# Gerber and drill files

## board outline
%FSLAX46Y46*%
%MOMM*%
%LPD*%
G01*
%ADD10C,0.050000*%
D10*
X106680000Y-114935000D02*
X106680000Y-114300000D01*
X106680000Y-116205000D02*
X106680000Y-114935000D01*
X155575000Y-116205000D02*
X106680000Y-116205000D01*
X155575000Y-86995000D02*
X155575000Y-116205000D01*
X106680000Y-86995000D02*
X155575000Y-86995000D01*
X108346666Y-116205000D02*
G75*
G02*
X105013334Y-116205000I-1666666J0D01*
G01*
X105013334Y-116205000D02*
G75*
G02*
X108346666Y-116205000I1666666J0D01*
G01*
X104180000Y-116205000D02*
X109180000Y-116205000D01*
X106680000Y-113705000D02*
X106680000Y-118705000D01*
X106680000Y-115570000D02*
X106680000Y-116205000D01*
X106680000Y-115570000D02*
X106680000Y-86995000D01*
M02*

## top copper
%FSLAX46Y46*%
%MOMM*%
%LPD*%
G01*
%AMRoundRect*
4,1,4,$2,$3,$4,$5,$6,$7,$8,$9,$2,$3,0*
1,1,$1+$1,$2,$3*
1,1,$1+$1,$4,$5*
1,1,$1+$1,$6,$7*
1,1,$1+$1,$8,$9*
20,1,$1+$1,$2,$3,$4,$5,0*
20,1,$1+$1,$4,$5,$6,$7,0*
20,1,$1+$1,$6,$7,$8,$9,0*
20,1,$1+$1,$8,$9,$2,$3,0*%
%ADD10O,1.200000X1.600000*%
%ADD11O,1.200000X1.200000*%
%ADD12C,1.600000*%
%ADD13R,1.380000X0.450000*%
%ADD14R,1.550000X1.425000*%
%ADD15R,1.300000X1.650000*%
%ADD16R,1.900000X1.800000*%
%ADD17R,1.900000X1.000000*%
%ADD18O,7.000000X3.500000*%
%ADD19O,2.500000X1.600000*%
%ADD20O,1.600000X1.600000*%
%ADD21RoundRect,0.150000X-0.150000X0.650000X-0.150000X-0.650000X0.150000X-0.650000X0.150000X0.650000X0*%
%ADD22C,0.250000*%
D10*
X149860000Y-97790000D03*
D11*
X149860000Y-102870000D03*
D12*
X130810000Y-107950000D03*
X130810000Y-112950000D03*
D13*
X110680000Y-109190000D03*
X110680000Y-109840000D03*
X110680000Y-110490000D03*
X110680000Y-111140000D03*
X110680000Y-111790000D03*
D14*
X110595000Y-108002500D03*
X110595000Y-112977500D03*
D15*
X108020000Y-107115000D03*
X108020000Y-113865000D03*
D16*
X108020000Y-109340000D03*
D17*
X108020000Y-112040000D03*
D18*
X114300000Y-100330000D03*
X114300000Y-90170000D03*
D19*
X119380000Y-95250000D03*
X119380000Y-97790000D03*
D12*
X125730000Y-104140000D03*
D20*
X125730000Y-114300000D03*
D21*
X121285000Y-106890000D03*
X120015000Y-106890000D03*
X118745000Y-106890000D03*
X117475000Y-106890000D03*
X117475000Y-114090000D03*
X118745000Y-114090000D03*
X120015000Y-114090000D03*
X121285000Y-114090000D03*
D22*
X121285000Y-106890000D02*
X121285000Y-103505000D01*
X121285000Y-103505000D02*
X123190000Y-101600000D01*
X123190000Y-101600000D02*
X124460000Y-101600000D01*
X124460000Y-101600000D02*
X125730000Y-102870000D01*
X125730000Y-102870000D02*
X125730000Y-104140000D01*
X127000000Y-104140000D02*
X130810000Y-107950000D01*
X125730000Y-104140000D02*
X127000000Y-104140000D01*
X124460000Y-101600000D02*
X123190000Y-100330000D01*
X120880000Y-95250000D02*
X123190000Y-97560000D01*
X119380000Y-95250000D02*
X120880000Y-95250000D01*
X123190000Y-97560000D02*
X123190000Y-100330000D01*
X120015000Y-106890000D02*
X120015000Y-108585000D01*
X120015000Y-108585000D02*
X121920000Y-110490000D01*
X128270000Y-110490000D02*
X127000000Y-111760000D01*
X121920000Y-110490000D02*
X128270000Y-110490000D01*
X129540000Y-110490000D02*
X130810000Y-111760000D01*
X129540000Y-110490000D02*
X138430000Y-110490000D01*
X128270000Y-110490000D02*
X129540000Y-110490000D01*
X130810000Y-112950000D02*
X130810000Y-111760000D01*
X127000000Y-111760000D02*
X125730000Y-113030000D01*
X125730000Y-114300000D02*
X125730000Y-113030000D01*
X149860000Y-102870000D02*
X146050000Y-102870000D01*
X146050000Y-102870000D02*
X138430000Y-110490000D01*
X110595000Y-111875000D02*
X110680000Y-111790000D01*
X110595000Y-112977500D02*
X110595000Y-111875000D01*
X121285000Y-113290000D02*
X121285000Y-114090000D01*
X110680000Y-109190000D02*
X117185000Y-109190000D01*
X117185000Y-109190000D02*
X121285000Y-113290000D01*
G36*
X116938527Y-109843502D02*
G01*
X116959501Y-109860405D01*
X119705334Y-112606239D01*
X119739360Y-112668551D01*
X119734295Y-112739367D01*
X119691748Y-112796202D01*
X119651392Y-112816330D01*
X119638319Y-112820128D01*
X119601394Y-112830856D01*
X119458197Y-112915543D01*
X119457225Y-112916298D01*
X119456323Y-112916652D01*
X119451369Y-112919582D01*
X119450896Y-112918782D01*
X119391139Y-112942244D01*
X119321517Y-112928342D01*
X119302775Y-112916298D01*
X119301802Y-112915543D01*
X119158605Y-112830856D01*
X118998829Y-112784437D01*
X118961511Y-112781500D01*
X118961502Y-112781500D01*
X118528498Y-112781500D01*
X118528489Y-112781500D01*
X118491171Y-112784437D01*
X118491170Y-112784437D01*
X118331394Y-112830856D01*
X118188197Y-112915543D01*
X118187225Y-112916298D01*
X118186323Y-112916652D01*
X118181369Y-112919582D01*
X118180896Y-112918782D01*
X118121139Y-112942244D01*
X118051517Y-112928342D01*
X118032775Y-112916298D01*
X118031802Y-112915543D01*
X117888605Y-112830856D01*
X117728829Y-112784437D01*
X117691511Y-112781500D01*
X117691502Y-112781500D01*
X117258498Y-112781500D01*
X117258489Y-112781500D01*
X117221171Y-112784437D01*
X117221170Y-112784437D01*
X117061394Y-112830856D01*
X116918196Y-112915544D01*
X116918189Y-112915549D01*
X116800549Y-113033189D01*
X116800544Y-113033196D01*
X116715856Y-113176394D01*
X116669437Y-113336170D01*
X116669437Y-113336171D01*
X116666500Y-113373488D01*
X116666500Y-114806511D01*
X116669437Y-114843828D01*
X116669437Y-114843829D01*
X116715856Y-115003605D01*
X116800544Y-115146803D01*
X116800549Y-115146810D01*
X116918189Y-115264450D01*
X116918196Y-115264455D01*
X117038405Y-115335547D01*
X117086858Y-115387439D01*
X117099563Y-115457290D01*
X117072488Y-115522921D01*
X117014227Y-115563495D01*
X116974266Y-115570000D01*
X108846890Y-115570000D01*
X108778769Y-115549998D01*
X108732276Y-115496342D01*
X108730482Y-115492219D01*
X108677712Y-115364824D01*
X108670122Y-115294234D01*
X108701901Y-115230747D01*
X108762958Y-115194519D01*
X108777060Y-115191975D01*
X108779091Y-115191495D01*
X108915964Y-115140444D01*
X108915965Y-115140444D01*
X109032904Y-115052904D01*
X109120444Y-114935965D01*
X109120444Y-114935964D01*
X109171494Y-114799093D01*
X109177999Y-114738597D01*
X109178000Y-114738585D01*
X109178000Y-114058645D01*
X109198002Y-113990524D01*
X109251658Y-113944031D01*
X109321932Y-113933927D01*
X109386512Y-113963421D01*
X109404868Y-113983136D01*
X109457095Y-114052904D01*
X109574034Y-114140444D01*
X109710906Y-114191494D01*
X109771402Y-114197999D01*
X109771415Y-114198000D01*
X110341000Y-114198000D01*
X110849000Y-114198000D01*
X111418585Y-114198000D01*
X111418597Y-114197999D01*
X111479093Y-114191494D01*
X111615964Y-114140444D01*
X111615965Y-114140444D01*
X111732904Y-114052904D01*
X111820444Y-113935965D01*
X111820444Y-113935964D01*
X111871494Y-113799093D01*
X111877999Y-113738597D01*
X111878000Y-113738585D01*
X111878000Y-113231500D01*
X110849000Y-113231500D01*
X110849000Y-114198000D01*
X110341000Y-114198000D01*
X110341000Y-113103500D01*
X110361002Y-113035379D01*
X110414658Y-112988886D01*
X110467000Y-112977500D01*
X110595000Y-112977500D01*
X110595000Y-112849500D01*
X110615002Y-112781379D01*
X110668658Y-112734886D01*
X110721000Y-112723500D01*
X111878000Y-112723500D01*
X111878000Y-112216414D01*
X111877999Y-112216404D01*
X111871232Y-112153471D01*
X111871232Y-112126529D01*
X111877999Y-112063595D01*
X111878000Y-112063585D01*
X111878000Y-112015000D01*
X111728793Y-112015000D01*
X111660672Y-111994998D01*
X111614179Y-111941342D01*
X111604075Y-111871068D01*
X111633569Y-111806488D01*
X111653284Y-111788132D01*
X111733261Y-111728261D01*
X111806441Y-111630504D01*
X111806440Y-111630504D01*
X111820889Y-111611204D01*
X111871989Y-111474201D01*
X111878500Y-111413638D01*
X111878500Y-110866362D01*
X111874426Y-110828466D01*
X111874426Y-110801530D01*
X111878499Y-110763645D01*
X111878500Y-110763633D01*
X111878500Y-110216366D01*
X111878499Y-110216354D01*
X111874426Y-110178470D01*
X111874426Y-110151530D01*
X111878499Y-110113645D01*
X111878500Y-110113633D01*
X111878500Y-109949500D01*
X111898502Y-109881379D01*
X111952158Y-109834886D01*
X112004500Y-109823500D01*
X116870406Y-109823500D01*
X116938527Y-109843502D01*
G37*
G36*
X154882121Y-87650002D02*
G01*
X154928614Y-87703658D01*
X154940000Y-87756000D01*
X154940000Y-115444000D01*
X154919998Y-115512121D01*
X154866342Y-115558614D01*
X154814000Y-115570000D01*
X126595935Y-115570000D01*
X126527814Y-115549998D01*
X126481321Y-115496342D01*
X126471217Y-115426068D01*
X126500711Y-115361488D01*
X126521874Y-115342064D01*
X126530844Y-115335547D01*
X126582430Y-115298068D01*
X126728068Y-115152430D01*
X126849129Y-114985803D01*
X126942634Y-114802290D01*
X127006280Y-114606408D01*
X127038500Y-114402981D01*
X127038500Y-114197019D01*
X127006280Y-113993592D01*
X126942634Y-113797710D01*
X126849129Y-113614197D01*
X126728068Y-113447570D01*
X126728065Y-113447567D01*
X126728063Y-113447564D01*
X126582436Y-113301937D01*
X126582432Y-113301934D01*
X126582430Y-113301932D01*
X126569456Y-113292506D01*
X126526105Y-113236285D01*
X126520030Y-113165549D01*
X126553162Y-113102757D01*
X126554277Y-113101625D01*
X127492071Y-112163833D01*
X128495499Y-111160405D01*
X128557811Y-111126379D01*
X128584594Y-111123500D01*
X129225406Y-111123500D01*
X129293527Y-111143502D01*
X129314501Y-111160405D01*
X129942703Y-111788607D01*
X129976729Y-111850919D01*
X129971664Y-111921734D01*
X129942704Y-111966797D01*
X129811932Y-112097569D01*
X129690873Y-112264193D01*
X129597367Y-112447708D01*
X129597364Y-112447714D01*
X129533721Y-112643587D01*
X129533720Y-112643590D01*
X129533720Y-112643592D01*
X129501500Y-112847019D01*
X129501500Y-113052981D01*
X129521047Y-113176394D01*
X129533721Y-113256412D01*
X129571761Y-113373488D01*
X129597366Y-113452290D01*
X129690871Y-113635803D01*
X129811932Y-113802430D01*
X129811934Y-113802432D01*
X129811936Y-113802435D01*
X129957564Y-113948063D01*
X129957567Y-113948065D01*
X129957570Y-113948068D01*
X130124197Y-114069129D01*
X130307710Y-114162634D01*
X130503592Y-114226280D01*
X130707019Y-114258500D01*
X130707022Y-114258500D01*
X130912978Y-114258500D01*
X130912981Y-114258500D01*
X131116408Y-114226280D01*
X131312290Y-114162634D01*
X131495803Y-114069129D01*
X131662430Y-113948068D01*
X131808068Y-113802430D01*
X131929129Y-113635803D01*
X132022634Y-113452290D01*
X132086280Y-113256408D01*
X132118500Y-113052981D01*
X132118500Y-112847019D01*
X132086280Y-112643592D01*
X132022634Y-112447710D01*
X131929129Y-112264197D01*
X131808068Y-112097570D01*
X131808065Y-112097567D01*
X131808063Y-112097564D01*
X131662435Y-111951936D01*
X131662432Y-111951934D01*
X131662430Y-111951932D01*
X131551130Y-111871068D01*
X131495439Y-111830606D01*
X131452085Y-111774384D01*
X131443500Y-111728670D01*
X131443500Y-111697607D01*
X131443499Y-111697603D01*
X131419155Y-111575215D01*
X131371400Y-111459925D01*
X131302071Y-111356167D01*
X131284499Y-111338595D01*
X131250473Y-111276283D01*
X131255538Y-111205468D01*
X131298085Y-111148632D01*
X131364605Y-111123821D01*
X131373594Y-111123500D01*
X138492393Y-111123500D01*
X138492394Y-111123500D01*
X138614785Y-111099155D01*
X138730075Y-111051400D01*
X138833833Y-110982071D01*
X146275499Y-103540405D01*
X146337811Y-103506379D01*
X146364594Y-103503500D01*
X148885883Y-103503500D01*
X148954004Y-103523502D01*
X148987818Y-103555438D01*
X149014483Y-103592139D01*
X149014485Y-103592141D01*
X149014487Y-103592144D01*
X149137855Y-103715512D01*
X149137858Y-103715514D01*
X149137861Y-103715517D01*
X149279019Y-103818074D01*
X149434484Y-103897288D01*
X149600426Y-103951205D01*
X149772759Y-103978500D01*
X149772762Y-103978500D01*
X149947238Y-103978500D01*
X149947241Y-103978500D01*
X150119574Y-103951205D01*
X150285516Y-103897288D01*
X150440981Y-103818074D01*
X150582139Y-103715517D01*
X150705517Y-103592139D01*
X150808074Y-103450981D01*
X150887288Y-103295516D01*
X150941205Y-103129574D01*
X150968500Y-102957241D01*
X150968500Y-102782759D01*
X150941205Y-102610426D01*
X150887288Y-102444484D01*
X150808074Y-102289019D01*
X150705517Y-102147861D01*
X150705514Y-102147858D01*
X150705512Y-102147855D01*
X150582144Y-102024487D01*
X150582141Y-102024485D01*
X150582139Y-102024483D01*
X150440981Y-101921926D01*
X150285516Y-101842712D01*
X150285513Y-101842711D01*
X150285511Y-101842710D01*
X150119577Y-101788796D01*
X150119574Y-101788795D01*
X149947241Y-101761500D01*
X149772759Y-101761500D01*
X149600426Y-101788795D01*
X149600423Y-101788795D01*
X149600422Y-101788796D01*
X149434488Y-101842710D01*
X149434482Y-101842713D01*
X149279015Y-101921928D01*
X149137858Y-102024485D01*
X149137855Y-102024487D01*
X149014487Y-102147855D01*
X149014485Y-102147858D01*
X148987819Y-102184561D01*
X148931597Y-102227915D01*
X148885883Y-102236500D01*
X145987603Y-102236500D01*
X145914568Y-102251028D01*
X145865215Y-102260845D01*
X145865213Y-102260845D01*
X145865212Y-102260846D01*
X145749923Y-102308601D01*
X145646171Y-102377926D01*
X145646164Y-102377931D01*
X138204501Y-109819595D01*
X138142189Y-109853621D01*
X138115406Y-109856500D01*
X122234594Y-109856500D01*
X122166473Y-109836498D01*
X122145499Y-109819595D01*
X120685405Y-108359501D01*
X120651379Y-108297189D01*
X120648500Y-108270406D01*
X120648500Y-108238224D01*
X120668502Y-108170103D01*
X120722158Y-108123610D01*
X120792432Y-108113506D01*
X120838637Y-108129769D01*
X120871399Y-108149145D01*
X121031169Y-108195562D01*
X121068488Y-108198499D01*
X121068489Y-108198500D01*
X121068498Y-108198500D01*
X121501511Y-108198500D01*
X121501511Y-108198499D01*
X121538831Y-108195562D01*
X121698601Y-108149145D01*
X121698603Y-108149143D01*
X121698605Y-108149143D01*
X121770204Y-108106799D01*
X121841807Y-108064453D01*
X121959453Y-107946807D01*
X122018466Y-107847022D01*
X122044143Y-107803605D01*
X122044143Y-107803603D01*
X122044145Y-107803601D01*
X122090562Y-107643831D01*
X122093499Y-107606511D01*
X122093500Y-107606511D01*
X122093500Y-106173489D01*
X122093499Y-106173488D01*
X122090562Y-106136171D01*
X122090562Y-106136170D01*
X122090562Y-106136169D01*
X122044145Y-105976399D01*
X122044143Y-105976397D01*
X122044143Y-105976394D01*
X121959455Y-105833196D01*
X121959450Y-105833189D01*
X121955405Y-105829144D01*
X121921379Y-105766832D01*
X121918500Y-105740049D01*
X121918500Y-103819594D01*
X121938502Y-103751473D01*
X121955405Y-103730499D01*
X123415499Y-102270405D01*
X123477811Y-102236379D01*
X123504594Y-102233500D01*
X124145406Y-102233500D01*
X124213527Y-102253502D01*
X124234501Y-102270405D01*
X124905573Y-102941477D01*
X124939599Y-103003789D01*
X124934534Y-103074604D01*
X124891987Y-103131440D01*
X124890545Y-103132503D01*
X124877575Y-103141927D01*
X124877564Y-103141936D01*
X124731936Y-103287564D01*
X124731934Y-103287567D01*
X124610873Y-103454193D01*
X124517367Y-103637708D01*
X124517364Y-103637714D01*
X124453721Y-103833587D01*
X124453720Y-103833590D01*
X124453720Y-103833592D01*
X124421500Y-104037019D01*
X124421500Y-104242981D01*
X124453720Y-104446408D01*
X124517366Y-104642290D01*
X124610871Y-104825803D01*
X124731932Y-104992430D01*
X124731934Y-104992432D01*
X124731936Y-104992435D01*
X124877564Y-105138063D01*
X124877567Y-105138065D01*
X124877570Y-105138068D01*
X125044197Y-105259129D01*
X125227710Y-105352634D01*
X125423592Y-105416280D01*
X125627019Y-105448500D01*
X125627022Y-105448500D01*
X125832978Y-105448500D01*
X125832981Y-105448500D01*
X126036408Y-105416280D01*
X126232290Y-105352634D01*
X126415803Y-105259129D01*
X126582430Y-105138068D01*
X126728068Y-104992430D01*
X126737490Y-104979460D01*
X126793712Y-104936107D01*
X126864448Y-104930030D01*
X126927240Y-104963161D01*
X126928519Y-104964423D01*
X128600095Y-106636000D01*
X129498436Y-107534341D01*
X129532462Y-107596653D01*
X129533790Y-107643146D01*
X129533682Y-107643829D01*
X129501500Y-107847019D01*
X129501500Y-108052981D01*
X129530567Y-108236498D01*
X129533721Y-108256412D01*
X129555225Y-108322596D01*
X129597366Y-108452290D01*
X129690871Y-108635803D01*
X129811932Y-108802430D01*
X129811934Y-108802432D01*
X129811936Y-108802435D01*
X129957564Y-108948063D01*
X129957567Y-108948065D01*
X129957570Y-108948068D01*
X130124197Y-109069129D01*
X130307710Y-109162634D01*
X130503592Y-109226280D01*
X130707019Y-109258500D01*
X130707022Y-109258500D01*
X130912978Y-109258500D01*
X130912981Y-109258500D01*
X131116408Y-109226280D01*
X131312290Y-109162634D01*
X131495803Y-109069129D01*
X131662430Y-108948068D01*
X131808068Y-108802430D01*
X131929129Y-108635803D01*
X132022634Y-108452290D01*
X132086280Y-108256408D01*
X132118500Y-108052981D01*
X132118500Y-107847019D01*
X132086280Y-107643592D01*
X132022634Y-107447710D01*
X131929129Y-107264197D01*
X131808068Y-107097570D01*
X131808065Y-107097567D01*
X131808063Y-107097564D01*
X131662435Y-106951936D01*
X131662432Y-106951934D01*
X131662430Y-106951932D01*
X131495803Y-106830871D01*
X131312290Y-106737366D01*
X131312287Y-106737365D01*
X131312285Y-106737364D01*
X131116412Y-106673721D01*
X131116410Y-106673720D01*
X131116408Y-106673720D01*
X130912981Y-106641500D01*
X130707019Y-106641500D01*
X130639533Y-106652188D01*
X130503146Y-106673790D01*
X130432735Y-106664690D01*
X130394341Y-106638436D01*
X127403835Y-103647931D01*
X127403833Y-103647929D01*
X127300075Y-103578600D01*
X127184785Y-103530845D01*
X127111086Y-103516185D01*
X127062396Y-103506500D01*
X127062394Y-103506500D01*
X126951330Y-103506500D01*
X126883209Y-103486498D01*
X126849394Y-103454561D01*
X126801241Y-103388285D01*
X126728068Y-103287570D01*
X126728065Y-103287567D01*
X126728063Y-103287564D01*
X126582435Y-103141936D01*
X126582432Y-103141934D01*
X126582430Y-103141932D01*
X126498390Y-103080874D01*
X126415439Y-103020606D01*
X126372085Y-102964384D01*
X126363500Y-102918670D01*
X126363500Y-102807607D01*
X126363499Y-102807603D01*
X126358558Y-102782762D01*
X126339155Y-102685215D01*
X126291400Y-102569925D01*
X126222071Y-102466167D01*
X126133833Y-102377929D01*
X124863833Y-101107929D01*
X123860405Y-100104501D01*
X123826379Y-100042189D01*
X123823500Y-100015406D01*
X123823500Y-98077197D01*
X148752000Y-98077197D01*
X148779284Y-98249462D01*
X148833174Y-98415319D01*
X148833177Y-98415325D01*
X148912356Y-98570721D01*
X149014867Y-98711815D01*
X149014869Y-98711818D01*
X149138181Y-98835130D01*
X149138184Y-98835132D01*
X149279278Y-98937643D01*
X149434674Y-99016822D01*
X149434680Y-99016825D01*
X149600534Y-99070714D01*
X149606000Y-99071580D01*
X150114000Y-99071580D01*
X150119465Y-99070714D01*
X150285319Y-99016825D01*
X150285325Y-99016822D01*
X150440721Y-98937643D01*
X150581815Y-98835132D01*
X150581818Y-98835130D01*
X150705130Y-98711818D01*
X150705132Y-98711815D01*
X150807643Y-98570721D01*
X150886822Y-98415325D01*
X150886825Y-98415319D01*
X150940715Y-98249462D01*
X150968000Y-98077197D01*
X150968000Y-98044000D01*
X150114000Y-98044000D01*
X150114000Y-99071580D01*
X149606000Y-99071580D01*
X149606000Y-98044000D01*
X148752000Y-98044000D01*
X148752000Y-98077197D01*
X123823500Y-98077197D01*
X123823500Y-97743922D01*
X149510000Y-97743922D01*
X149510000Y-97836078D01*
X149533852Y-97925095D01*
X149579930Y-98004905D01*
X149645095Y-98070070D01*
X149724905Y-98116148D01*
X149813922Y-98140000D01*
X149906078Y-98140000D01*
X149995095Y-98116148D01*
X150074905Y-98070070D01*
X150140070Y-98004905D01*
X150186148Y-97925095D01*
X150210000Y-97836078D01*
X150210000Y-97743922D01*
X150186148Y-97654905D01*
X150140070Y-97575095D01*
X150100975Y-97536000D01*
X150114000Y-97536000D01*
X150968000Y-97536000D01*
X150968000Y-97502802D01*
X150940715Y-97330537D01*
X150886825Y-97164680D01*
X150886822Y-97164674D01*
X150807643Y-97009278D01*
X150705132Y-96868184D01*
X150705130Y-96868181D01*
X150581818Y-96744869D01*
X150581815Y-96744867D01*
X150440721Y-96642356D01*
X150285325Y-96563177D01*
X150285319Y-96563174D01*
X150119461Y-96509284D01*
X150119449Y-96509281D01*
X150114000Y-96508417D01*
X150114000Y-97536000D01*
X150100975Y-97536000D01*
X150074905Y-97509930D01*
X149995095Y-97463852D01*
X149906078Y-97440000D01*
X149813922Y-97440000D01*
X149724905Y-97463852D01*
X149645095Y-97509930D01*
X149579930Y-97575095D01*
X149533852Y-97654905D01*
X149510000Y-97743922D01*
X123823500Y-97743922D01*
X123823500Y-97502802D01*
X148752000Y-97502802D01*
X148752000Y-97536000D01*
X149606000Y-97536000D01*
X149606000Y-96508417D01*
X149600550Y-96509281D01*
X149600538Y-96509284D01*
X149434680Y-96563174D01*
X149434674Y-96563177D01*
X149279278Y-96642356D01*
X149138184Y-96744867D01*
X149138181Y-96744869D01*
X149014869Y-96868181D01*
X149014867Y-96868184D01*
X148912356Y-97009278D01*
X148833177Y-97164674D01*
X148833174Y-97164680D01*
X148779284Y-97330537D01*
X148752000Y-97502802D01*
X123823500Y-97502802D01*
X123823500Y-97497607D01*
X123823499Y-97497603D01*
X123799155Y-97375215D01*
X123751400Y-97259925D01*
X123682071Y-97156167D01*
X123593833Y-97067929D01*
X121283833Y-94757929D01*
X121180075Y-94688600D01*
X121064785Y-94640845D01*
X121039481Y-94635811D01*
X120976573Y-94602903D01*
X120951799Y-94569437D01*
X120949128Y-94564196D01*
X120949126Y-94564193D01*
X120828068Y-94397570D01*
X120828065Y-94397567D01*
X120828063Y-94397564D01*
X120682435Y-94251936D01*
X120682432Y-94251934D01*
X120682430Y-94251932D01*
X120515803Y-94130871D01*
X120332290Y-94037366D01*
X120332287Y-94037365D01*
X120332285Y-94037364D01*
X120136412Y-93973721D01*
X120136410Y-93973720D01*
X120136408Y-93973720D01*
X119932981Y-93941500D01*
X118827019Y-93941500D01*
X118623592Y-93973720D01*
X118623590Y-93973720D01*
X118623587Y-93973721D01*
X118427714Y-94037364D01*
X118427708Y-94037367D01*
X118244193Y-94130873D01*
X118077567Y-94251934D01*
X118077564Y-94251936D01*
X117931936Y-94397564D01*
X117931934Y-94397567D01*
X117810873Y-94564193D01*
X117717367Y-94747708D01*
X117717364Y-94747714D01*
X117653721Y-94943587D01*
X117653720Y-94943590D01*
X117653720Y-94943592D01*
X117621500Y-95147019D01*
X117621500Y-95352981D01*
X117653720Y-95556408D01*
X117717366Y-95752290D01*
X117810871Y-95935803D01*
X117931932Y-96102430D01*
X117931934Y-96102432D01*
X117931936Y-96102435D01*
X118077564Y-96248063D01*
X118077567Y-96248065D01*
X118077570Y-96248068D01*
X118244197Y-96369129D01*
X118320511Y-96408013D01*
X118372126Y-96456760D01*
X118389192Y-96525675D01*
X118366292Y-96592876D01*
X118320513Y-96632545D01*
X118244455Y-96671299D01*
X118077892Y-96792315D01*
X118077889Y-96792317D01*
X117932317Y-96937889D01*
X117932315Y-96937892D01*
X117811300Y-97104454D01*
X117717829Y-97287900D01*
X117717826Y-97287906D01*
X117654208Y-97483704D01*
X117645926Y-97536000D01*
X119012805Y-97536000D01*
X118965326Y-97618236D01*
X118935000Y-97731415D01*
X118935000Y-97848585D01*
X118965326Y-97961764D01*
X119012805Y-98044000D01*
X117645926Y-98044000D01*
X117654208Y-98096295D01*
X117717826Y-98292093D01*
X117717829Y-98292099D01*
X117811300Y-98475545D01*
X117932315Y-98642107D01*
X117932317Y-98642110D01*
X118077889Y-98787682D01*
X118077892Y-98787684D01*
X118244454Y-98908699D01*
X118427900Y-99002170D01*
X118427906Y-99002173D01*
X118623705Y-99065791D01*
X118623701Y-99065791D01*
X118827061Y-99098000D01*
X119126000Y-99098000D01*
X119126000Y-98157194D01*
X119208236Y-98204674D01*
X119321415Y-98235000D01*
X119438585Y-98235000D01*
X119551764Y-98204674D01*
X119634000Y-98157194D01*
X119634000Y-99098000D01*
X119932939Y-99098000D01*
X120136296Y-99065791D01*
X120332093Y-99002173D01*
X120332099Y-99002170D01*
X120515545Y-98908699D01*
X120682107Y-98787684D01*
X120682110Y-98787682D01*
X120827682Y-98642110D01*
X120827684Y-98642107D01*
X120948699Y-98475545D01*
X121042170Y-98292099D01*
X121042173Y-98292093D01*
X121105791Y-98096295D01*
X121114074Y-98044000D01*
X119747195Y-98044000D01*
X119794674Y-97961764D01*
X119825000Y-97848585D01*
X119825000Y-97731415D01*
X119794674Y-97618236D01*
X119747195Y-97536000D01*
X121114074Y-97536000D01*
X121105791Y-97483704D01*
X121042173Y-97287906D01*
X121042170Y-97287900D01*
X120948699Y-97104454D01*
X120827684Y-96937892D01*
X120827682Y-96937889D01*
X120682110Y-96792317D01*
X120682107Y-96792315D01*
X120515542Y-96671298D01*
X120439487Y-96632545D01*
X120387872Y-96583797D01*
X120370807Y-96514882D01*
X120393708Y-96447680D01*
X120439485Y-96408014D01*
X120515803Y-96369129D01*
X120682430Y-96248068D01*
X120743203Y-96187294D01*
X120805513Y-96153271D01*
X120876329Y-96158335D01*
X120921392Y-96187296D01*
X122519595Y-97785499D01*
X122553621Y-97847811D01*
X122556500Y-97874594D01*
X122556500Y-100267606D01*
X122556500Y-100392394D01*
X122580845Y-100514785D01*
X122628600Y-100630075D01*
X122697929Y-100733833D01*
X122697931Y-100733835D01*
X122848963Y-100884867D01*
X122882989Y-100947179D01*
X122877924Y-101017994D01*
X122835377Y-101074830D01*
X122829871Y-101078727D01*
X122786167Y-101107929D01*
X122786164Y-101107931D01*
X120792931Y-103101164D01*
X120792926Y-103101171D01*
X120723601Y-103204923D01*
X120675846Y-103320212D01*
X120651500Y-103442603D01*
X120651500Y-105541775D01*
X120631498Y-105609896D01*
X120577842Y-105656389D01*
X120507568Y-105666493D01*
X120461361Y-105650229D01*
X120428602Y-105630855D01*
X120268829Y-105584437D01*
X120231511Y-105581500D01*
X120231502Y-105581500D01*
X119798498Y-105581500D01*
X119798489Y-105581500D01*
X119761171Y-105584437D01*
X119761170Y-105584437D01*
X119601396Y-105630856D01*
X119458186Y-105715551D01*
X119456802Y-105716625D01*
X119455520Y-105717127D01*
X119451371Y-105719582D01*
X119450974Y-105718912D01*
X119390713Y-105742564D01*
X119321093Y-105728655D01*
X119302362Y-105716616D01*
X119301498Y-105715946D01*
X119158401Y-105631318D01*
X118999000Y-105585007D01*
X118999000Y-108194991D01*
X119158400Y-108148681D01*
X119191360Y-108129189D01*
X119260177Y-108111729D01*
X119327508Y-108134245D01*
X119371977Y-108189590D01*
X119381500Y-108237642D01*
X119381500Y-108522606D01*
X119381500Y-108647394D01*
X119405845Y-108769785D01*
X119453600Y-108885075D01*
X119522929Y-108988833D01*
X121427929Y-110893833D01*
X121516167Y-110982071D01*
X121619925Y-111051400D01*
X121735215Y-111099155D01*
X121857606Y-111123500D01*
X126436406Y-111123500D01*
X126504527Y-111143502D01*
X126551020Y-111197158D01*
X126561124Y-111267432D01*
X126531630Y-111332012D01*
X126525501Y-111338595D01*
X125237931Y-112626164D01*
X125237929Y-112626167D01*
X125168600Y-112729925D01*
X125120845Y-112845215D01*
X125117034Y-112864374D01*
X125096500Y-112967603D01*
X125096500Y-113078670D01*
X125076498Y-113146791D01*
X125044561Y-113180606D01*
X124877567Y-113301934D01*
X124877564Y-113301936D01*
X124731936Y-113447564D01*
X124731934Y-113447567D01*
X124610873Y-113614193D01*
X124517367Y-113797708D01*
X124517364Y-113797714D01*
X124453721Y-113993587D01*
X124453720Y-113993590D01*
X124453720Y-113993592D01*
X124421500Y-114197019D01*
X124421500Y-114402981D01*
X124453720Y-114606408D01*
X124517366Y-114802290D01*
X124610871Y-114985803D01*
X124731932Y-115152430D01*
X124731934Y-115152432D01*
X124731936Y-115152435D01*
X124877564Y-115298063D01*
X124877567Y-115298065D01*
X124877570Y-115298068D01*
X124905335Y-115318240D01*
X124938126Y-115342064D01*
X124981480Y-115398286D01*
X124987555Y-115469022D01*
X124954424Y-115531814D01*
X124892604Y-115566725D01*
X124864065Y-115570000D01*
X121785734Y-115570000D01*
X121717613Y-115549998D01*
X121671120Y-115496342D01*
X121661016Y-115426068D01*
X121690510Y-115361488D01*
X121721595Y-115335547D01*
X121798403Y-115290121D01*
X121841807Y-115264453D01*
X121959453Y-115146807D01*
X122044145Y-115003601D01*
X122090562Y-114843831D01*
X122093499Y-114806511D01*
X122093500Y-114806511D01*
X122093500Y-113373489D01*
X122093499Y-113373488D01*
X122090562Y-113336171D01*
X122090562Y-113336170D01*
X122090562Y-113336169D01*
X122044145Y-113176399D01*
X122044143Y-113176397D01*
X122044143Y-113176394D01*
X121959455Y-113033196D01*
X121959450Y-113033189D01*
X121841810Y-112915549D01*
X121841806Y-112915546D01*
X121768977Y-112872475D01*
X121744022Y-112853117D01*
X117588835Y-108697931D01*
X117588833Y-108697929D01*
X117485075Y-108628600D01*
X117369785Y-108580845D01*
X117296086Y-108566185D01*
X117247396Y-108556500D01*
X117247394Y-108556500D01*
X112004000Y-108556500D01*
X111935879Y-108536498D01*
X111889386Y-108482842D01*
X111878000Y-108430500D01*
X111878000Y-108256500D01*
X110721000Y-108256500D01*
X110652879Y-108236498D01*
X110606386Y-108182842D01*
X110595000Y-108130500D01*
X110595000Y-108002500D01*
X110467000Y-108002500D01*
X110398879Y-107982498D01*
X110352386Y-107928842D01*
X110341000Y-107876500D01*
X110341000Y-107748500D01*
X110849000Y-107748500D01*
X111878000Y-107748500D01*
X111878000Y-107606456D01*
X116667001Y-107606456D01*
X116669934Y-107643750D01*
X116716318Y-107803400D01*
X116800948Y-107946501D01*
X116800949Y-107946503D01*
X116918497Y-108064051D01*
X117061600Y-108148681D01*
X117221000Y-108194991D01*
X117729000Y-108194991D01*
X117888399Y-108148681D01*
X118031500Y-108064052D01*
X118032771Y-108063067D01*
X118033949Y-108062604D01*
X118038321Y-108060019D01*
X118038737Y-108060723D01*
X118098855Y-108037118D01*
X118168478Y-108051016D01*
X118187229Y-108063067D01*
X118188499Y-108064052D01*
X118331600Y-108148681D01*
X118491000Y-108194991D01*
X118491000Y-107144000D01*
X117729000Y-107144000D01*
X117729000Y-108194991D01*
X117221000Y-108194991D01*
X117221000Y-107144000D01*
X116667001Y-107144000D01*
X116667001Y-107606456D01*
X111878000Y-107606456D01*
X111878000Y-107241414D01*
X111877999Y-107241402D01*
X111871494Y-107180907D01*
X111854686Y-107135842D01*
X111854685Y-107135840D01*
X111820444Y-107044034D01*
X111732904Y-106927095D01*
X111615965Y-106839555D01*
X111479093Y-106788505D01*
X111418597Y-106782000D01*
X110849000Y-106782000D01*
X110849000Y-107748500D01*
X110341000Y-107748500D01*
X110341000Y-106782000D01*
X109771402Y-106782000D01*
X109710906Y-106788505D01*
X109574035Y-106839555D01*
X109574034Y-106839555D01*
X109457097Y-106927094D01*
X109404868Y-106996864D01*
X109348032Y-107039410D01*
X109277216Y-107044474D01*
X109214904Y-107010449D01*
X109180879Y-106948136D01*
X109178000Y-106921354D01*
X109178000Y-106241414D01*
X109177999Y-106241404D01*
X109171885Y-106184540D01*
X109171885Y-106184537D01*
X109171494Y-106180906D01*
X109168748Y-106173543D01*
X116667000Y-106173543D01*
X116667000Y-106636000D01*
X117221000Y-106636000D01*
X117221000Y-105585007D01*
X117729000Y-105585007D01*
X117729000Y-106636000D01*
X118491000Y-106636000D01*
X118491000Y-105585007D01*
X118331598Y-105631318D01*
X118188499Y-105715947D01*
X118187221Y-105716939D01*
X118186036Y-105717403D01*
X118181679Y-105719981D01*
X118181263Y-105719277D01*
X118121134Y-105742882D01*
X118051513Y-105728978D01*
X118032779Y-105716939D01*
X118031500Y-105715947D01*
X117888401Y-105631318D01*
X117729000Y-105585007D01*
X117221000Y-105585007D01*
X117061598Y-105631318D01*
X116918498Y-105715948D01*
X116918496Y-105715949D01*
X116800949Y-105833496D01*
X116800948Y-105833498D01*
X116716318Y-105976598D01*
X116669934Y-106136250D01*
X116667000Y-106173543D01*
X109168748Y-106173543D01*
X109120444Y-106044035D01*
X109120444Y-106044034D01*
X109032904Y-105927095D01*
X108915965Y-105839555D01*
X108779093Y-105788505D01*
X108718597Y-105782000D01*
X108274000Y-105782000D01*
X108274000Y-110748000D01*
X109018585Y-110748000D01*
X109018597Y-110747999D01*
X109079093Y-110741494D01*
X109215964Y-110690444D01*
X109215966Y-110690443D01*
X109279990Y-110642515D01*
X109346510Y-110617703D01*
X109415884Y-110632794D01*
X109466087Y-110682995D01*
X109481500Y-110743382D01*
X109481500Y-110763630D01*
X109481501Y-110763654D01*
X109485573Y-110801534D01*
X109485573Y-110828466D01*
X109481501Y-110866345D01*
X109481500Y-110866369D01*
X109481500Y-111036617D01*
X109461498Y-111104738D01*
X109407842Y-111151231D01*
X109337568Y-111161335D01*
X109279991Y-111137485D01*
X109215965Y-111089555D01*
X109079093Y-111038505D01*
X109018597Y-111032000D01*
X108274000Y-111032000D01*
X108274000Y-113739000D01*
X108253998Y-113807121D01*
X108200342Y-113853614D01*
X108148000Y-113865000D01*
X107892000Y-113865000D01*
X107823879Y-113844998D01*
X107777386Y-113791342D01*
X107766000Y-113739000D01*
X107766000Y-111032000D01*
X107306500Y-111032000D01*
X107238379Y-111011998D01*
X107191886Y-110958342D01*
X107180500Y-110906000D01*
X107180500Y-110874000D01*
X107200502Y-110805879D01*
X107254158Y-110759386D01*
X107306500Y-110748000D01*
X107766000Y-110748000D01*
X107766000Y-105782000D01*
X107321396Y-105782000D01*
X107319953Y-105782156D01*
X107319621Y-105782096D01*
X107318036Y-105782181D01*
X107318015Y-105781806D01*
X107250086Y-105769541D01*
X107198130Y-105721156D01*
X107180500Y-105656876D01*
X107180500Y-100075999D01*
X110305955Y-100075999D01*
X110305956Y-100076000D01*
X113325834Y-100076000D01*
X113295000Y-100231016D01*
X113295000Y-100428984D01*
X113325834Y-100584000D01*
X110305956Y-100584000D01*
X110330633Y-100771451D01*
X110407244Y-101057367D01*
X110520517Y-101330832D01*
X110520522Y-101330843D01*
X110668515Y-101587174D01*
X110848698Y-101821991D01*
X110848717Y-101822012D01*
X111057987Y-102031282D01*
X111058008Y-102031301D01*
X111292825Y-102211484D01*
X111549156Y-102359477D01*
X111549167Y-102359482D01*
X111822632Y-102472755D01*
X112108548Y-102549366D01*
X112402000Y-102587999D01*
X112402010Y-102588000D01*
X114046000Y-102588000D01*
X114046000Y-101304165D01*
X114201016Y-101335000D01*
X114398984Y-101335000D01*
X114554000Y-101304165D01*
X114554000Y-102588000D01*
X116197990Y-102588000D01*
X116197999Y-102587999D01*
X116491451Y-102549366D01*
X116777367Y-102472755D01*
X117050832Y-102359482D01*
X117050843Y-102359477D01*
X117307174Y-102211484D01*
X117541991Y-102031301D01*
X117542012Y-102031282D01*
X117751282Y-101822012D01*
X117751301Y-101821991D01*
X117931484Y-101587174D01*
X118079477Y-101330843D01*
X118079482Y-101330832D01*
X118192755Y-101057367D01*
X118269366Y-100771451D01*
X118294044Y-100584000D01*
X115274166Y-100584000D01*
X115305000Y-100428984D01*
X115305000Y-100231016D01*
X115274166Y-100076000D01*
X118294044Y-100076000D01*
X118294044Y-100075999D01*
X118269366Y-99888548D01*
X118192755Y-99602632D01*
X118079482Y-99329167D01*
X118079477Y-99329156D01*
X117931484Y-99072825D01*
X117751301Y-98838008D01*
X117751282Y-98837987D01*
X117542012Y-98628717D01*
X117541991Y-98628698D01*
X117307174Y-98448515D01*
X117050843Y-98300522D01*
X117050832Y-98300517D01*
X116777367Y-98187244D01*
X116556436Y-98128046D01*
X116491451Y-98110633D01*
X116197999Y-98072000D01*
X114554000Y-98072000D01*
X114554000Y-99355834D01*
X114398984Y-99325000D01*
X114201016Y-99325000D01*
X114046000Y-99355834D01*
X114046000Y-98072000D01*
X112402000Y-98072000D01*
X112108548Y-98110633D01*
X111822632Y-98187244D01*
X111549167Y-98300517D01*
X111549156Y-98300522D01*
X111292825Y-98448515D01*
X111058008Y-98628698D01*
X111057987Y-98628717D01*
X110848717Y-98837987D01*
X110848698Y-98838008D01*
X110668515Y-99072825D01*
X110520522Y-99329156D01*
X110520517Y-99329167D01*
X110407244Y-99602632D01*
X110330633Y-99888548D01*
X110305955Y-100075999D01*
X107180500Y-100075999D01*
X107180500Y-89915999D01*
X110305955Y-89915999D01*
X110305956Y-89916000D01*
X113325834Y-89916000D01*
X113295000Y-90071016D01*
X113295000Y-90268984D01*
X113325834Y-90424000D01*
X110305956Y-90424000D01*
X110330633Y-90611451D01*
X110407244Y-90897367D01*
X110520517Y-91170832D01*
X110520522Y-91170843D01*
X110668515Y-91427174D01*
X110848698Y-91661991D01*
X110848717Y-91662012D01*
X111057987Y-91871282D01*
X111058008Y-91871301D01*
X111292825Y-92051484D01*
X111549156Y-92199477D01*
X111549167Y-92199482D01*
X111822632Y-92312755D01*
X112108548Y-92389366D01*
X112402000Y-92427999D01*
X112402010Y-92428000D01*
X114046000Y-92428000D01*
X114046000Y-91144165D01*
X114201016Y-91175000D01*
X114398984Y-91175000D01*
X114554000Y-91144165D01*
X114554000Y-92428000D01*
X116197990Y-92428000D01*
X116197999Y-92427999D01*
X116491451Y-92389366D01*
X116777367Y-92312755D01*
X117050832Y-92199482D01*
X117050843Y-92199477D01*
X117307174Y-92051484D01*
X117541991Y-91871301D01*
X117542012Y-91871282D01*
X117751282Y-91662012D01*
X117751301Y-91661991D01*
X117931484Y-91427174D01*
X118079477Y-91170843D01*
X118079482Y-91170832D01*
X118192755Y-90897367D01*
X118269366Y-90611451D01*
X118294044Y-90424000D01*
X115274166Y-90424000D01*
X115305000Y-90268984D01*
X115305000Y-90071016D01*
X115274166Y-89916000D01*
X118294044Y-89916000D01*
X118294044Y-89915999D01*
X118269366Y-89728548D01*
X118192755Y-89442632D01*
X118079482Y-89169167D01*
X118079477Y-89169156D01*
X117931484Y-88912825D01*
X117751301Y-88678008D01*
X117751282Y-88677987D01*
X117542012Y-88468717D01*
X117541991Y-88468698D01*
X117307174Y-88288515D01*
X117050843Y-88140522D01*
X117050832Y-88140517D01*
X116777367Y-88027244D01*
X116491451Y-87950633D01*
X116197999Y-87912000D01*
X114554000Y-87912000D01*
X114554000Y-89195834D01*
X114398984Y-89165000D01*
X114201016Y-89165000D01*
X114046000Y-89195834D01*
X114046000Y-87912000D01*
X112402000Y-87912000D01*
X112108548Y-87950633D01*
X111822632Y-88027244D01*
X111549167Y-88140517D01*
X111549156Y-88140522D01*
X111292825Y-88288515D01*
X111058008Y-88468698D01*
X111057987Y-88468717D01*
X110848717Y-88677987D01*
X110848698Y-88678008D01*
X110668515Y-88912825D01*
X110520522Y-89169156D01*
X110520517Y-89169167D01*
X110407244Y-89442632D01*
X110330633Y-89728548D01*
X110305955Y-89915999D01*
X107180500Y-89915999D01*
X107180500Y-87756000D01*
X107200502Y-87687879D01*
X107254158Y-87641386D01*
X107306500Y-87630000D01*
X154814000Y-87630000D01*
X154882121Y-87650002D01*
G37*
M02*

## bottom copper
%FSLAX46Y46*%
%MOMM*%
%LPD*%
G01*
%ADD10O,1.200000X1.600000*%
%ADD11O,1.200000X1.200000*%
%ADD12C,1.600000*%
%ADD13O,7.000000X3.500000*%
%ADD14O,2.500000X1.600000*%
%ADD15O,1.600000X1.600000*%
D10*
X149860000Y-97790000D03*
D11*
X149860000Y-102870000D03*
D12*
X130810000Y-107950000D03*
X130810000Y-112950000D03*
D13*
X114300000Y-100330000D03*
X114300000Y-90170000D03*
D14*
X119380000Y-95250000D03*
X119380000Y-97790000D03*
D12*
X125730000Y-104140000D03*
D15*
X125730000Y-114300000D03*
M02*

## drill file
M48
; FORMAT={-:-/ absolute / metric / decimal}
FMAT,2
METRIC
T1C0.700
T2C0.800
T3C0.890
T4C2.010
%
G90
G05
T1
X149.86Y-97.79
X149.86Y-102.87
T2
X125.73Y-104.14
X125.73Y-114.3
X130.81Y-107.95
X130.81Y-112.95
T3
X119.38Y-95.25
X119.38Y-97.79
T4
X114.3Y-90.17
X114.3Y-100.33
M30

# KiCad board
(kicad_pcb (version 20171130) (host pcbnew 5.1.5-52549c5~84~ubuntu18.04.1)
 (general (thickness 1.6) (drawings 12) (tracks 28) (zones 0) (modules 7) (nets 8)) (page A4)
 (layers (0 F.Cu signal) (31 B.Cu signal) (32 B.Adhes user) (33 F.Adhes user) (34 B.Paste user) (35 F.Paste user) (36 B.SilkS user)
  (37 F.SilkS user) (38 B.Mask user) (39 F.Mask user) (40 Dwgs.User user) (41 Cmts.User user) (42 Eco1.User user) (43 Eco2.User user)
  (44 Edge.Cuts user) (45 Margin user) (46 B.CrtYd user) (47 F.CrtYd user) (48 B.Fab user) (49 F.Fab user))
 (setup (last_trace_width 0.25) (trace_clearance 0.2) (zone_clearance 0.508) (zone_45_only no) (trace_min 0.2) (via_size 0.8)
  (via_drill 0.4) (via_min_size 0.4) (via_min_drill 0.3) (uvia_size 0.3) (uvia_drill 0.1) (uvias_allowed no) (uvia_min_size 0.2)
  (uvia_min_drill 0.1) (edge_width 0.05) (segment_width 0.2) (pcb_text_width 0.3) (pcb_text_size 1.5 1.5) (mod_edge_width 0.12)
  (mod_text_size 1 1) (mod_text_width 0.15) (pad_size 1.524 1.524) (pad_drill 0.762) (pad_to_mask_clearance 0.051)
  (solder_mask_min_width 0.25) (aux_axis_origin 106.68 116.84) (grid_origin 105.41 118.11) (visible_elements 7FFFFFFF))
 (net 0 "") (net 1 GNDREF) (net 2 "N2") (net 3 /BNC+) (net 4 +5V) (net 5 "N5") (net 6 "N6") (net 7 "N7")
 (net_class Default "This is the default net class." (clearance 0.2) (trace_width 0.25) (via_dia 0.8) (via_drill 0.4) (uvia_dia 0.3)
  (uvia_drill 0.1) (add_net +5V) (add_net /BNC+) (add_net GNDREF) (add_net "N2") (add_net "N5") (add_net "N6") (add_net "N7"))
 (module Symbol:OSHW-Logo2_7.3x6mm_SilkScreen (layer F.Cu) (at 151.13 90.805)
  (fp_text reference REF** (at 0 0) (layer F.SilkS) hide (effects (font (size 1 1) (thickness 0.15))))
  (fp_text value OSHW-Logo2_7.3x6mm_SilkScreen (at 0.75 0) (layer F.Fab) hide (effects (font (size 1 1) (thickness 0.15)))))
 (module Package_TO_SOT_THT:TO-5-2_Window (layer F.Cu) (at 149.86 97.79 270)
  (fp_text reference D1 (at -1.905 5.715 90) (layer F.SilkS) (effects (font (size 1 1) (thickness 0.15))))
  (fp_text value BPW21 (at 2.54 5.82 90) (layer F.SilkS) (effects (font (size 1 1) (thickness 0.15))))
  (pad 1 thru_hole oval (at 0 0 270) (size 1.6 1.2) (drill 0.7) (layers *.Cu *.Mask) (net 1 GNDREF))
  (pad 2 thru_hole oval (at 5.08 0 270) (size 1.2 1.2) (drill 0.7) (layers *.Cu *.Mask) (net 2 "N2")))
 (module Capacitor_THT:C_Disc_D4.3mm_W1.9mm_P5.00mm (layer F.Cu) (at 130.81 107.95 270)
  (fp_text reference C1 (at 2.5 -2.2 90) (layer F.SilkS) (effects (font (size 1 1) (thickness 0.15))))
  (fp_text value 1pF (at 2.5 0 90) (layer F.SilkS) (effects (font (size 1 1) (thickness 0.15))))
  (pad 1 thru_hole circle (at 0 0 270) (size 1.6 1.6) (drill 0.8) (layers *.Cu *.Mask) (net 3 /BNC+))
  (pad 2 thru_hole circle (at 5 0 270) (size 1.6 1.6) (drill 0.8) (layers *.Cu *.Mask) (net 2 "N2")))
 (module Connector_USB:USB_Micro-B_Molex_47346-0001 (layer F.Cu) (at 109.22 110.49 270)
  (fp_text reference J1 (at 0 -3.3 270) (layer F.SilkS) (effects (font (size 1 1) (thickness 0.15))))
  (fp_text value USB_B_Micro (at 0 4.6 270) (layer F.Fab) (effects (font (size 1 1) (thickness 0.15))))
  (pad 1 smd rect (at -1.3 -1.46 270) (size 0.45 1.38) (layers F.Cu F.Paste F.Mask) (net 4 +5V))
  (pad 2 smd rect (at -0.65 -1.46 270) (size 0.45 1.38) (layers F.Cu F.Paste F.Mask) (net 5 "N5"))
  (pad 3 smd rect (at 0 -1.46 270) (size 0.45 1.38) (layers F.Cu F.Paste F.Mask) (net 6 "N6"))
  (pad 4 smd rect (at 0.65 -1.46 270) (size 0.45 1.38) (layers F.Cu F.Paste F.Mask) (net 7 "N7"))
  (pad 5 smd rect (at 1.3 -1.46 270) (size 0.45 1.38) (layers F.Cu F.Paste F.Mask) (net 1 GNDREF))
  (pad 6 smd rect (at -2.4875 -1.375 270) (size 1.425 1.55) (layers F.Cu F.Paste F.Mask) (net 1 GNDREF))
  (pad 6 smd rect (at 2.4875 -1.375 270) (size 1.425 1.55) (layers F.Cu F.Paste F.Mask) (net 1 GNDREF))
  (pad 6 smd rect (at -3.375 1.2 270) (size 1.65 1.3) (layers F.Cu F.Paste F.Mask) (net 1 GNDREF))
  (pad 6 smd rect (at 3.375 1.2 270) (size 1.65 1.3) (layers F.Cu F.Paste F.Mask) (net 1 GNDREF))
  (pad 6 smd rect (at -1.15 1.2 270) (size 1.8 1.9) (layers F.Cu F.Paste F.Mask) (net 1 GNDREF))
  (pad 6 smd rect (at 1.55 1.2 270) (size 1 1.9) (layers F.Cu F.Paste F.Mask) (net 1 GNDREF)))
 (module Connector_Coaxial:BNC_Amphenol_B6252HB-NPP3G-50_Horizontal (layer F.Cu) (at 119.38 95.25 90)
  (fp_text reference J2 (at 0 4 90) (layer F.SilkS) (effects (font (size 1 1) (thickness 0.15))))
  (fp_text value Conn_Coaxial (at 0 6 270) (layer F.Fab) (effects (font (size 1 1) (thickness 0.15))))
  (pad 2 thru_hole oval (at -5.08 -5.08 90) (size 3.5 7) (drill 2.01) (layers *.Cu *.Mask) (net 1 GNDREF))
  (pad 2 thru_hole oval (at 5.08 -5.08 90) (size 3.5 7) (drill 2.01) (layers *.Cu *.Mask) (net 1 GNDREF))
  (pad 1 thru_hole oval (at 0 0 90) (size 1.6 2.5) (drill 0.89) (layers *.Cu *.Mask) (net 3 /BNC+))
  (pad 2 thru_hole oval (at -2.54 0 90) (size 1.6 2.5) (drill 0.89) (layers *.Cu *.Mask) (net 1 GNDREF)))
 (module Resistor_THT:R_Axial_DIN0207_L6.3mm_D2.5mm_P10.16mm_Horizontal (layer F.Cu) (at 125.73 104.14 270)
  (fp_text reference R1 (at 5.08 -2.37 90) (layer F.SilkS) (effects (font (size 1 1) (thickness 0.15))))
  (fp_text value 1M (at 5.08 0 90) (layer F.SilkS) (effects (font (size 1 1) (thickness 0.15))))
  (pad 1 thru_hole circle (at 0 0 270) (size 1.6 1.6) (drill 0.8) (layers *.Cu *.Mask) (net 3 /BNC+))
  (pad 2 thru_hole oval (at 10.16 0 270) (size 1.6 1.6) (drill 0.8) (layers *.Cu *.Mask) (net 2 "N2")))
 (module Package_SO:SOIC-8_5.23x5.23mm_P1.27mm (layer F.Cu) (at 119.38 110.49 270)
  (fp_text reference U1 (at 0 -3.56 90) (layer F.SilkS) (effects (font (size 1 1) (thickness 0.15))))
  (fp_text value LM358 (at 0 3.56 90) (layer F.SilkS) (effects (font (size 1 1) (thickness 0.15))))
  (pad 1 smd roundrect (at -3.6 -1.905 270) (size 1.6 0.6) (layers F.Cu F.Paste F.Mask) (roundrect_rratio 0.25) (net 3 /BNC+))
  (pad 2 smd roundrect (at -3.6 -0.635 270) (size 1.6 0.6) (layers F.Cu F.Paste F.Mask) (roundrect_rratio 0.25) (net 2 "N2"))
  (pad 3 smd roundrect (at -3.6 0.635 270) (size 1.6 0.6) (layers F.Cu F.Paste F.Mask) (roundrect_rratio 0.25) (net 1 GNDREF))
  (pad 4 smd roundrect (at -3.6 1.905 270) (size 1.6 0.6) (layers F.Cu F.Paste F.Mask) (roundrect_rratio 0.25) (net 1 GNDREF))
  (pad 5 smd roundrect (at 3.6 1.905 270) (size 1.6 0.6) (layers F.Cu F.Paste F.Mask) (roundrect_rratio 0.25))
  (pad 6 smd roundrect (at 3.6 0.635 270) (size 1.6 0.6) (layers F.Cu F.Paste F.Mask) (roundrect_rratio 0.25))
  (pad 7 smd roundrect (at 3.6 -0.635 270) (size 1.6 0.6) (layers F.Cu F.Paste F.Mask) (roundrect_rratio 0.25))
  (pad 8 smd roundrect (at 3.6 -1.905 270) (size 1.6 0.6) (layers F.Cu F.Paste F.Mask) (roundrect_rratio 0.25) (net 4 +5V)))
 (gr_line (start 106.68 114.935) (end 106.68 114.3) (layer Edge.Cuts) (width 0.05))
 (gr_line (start 106.68 116.205) (end 106.68 114.935) (layer Edge.Cuts) (width 0.05))
 (gr_line (start 155.575 116.205) (end 106.68 116.205) (layer Edge.Cuts) (width 0.05))
 (gr_line (start 155.575 86.995) (end 155.575 116.205) (layer Edge.Cuts) (width 0.05))
 (gr_line (start 106.68 86.995) (end 155.575 86.995) (layer Edge.Cuts) (width 0.05))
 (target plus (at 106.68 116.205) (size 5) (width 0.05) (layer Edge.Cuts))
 (gr_line (start 106.68 115.57) (end 106.68 116.205) (layer Edge.Cuts) (width 0.05))
 (gr_line (start 106.68 115.57) (end 106.68 86.995) (layer Edge.Cuts) (width 0.05))
 (segment (start 121.285 106.89) (end 121.285 103.505) (width 0.25) (layer F.Cu) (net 3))
 (segment (start 121.285 103.505) (end 123.19 101.6) (width 0.25) (layer F.Cu) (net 3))
 (segment (start 123.19 101.6) (end 124.46 101.6) (width 0.25) (layer F.Cu) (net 3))
 (segment (start 124.46 101.6) (end 125.73 102.87) (width 0.25) (layer F.Cu) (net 3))
 (segment (start 125.73 102.87) (end 125.73 104.14) (width 0.25) (layer F.Cu) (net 3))
 (segment (start 127 104.14) (end 130.81 107.95) (width 0.25) (layer F.Cu) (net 3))
 (segment (start 125.73 104.14) (end 127 104.14) (width 0.25) (layer F.Cu) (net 3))
 (segment (start 124.46 101.6) (end 123.19 100.33) (width 0.25) (layer F.Cu) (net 3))
 (segment (start 120.88 95.25) (end 123.19 97.56) (width 0.25) (layer F.Cu) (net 3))
 (segment (start 119.38 95.25) (end 120.88 95.25) (width 0.25) (layer F.Cu) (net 3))
 (segment (start 123.19 97.56) (end 123.19 100.33) (width 0.25) (layer F.Cu) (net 3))
 (segment (start 120.015 106.89) (end 120.015 108.585) (width 0.25) (layer F.Cu) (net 2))
 (segment (start 120.015 108.585) (end 121.92 110.49) (width 0.25) (layer F.Cu) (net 2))
 (segment (start 128.27 110.49) (end 127 111.76) (width 0.25) (layer F.Cu) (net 2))
 (segment (start 121.92 110.49) (end 128.27 110.49) (width 0.25) (layer F.Cu) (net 2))
 (segment (start 129.54 110.49) (end 130.81 111.76) (width 0.25) (layer F.Cu) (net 2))
 (segment (start 129.54 110.49) (end 138.43 110.49) (width 0.25) (layer F.Cu) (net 2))
 (segment (start 128.27 110.49) (end 129.54 110.49) (width 0.25) (layer F.Cu) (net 2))
 (segment (start 130.81 112.95) (end 130.81 111.76) (width 0.25) (layer F.Cu) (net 2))
 (segment (start 127 111.76) (end 125.73 113.03) (width 0.25) (layer F.Cu) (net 2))
 (segment (start 125.73 114.3) (end 125.73 113.03) (width 0.25) (layer F.Cu) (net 2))
 (segment (start 149.86 102.87) (end 146.05 102.87) (width 0.25) (layer F.Cu) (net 2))
 (segment (start 146.05 102.87) (end 138.43 110.49) (width 0.25) (layer F.Cu) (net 2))
 (segment (start 110.595 111.875) (end 110.68 111.79) (width 0.25) (layer F.Cu) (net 1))
 (segment (start 110.595 112.9775) (end 110.595 111.875) (width 0.25) (layer F.Cu) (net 1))
 (segment (start 121.285 113.29) (end 121.285 114.09) (width 0.25) (layer F.Cu) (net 4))
 (segment (start 110.68 109.19) (end 117.185 109.19) (width 0.25) (layer F.Cu) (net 4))
 (segment (start 117.185 109.19) (end 121.285 113.29) (width 0.25) (layer F.Cu) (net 4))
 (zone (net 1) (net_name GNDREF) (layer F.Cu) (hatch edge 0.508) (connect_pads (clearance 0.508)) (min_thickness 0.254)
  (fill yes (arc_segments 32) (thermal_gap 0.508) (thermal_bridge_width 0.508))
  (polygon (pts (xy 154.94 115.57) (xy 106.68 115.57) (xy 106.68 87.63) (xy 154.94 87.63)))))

